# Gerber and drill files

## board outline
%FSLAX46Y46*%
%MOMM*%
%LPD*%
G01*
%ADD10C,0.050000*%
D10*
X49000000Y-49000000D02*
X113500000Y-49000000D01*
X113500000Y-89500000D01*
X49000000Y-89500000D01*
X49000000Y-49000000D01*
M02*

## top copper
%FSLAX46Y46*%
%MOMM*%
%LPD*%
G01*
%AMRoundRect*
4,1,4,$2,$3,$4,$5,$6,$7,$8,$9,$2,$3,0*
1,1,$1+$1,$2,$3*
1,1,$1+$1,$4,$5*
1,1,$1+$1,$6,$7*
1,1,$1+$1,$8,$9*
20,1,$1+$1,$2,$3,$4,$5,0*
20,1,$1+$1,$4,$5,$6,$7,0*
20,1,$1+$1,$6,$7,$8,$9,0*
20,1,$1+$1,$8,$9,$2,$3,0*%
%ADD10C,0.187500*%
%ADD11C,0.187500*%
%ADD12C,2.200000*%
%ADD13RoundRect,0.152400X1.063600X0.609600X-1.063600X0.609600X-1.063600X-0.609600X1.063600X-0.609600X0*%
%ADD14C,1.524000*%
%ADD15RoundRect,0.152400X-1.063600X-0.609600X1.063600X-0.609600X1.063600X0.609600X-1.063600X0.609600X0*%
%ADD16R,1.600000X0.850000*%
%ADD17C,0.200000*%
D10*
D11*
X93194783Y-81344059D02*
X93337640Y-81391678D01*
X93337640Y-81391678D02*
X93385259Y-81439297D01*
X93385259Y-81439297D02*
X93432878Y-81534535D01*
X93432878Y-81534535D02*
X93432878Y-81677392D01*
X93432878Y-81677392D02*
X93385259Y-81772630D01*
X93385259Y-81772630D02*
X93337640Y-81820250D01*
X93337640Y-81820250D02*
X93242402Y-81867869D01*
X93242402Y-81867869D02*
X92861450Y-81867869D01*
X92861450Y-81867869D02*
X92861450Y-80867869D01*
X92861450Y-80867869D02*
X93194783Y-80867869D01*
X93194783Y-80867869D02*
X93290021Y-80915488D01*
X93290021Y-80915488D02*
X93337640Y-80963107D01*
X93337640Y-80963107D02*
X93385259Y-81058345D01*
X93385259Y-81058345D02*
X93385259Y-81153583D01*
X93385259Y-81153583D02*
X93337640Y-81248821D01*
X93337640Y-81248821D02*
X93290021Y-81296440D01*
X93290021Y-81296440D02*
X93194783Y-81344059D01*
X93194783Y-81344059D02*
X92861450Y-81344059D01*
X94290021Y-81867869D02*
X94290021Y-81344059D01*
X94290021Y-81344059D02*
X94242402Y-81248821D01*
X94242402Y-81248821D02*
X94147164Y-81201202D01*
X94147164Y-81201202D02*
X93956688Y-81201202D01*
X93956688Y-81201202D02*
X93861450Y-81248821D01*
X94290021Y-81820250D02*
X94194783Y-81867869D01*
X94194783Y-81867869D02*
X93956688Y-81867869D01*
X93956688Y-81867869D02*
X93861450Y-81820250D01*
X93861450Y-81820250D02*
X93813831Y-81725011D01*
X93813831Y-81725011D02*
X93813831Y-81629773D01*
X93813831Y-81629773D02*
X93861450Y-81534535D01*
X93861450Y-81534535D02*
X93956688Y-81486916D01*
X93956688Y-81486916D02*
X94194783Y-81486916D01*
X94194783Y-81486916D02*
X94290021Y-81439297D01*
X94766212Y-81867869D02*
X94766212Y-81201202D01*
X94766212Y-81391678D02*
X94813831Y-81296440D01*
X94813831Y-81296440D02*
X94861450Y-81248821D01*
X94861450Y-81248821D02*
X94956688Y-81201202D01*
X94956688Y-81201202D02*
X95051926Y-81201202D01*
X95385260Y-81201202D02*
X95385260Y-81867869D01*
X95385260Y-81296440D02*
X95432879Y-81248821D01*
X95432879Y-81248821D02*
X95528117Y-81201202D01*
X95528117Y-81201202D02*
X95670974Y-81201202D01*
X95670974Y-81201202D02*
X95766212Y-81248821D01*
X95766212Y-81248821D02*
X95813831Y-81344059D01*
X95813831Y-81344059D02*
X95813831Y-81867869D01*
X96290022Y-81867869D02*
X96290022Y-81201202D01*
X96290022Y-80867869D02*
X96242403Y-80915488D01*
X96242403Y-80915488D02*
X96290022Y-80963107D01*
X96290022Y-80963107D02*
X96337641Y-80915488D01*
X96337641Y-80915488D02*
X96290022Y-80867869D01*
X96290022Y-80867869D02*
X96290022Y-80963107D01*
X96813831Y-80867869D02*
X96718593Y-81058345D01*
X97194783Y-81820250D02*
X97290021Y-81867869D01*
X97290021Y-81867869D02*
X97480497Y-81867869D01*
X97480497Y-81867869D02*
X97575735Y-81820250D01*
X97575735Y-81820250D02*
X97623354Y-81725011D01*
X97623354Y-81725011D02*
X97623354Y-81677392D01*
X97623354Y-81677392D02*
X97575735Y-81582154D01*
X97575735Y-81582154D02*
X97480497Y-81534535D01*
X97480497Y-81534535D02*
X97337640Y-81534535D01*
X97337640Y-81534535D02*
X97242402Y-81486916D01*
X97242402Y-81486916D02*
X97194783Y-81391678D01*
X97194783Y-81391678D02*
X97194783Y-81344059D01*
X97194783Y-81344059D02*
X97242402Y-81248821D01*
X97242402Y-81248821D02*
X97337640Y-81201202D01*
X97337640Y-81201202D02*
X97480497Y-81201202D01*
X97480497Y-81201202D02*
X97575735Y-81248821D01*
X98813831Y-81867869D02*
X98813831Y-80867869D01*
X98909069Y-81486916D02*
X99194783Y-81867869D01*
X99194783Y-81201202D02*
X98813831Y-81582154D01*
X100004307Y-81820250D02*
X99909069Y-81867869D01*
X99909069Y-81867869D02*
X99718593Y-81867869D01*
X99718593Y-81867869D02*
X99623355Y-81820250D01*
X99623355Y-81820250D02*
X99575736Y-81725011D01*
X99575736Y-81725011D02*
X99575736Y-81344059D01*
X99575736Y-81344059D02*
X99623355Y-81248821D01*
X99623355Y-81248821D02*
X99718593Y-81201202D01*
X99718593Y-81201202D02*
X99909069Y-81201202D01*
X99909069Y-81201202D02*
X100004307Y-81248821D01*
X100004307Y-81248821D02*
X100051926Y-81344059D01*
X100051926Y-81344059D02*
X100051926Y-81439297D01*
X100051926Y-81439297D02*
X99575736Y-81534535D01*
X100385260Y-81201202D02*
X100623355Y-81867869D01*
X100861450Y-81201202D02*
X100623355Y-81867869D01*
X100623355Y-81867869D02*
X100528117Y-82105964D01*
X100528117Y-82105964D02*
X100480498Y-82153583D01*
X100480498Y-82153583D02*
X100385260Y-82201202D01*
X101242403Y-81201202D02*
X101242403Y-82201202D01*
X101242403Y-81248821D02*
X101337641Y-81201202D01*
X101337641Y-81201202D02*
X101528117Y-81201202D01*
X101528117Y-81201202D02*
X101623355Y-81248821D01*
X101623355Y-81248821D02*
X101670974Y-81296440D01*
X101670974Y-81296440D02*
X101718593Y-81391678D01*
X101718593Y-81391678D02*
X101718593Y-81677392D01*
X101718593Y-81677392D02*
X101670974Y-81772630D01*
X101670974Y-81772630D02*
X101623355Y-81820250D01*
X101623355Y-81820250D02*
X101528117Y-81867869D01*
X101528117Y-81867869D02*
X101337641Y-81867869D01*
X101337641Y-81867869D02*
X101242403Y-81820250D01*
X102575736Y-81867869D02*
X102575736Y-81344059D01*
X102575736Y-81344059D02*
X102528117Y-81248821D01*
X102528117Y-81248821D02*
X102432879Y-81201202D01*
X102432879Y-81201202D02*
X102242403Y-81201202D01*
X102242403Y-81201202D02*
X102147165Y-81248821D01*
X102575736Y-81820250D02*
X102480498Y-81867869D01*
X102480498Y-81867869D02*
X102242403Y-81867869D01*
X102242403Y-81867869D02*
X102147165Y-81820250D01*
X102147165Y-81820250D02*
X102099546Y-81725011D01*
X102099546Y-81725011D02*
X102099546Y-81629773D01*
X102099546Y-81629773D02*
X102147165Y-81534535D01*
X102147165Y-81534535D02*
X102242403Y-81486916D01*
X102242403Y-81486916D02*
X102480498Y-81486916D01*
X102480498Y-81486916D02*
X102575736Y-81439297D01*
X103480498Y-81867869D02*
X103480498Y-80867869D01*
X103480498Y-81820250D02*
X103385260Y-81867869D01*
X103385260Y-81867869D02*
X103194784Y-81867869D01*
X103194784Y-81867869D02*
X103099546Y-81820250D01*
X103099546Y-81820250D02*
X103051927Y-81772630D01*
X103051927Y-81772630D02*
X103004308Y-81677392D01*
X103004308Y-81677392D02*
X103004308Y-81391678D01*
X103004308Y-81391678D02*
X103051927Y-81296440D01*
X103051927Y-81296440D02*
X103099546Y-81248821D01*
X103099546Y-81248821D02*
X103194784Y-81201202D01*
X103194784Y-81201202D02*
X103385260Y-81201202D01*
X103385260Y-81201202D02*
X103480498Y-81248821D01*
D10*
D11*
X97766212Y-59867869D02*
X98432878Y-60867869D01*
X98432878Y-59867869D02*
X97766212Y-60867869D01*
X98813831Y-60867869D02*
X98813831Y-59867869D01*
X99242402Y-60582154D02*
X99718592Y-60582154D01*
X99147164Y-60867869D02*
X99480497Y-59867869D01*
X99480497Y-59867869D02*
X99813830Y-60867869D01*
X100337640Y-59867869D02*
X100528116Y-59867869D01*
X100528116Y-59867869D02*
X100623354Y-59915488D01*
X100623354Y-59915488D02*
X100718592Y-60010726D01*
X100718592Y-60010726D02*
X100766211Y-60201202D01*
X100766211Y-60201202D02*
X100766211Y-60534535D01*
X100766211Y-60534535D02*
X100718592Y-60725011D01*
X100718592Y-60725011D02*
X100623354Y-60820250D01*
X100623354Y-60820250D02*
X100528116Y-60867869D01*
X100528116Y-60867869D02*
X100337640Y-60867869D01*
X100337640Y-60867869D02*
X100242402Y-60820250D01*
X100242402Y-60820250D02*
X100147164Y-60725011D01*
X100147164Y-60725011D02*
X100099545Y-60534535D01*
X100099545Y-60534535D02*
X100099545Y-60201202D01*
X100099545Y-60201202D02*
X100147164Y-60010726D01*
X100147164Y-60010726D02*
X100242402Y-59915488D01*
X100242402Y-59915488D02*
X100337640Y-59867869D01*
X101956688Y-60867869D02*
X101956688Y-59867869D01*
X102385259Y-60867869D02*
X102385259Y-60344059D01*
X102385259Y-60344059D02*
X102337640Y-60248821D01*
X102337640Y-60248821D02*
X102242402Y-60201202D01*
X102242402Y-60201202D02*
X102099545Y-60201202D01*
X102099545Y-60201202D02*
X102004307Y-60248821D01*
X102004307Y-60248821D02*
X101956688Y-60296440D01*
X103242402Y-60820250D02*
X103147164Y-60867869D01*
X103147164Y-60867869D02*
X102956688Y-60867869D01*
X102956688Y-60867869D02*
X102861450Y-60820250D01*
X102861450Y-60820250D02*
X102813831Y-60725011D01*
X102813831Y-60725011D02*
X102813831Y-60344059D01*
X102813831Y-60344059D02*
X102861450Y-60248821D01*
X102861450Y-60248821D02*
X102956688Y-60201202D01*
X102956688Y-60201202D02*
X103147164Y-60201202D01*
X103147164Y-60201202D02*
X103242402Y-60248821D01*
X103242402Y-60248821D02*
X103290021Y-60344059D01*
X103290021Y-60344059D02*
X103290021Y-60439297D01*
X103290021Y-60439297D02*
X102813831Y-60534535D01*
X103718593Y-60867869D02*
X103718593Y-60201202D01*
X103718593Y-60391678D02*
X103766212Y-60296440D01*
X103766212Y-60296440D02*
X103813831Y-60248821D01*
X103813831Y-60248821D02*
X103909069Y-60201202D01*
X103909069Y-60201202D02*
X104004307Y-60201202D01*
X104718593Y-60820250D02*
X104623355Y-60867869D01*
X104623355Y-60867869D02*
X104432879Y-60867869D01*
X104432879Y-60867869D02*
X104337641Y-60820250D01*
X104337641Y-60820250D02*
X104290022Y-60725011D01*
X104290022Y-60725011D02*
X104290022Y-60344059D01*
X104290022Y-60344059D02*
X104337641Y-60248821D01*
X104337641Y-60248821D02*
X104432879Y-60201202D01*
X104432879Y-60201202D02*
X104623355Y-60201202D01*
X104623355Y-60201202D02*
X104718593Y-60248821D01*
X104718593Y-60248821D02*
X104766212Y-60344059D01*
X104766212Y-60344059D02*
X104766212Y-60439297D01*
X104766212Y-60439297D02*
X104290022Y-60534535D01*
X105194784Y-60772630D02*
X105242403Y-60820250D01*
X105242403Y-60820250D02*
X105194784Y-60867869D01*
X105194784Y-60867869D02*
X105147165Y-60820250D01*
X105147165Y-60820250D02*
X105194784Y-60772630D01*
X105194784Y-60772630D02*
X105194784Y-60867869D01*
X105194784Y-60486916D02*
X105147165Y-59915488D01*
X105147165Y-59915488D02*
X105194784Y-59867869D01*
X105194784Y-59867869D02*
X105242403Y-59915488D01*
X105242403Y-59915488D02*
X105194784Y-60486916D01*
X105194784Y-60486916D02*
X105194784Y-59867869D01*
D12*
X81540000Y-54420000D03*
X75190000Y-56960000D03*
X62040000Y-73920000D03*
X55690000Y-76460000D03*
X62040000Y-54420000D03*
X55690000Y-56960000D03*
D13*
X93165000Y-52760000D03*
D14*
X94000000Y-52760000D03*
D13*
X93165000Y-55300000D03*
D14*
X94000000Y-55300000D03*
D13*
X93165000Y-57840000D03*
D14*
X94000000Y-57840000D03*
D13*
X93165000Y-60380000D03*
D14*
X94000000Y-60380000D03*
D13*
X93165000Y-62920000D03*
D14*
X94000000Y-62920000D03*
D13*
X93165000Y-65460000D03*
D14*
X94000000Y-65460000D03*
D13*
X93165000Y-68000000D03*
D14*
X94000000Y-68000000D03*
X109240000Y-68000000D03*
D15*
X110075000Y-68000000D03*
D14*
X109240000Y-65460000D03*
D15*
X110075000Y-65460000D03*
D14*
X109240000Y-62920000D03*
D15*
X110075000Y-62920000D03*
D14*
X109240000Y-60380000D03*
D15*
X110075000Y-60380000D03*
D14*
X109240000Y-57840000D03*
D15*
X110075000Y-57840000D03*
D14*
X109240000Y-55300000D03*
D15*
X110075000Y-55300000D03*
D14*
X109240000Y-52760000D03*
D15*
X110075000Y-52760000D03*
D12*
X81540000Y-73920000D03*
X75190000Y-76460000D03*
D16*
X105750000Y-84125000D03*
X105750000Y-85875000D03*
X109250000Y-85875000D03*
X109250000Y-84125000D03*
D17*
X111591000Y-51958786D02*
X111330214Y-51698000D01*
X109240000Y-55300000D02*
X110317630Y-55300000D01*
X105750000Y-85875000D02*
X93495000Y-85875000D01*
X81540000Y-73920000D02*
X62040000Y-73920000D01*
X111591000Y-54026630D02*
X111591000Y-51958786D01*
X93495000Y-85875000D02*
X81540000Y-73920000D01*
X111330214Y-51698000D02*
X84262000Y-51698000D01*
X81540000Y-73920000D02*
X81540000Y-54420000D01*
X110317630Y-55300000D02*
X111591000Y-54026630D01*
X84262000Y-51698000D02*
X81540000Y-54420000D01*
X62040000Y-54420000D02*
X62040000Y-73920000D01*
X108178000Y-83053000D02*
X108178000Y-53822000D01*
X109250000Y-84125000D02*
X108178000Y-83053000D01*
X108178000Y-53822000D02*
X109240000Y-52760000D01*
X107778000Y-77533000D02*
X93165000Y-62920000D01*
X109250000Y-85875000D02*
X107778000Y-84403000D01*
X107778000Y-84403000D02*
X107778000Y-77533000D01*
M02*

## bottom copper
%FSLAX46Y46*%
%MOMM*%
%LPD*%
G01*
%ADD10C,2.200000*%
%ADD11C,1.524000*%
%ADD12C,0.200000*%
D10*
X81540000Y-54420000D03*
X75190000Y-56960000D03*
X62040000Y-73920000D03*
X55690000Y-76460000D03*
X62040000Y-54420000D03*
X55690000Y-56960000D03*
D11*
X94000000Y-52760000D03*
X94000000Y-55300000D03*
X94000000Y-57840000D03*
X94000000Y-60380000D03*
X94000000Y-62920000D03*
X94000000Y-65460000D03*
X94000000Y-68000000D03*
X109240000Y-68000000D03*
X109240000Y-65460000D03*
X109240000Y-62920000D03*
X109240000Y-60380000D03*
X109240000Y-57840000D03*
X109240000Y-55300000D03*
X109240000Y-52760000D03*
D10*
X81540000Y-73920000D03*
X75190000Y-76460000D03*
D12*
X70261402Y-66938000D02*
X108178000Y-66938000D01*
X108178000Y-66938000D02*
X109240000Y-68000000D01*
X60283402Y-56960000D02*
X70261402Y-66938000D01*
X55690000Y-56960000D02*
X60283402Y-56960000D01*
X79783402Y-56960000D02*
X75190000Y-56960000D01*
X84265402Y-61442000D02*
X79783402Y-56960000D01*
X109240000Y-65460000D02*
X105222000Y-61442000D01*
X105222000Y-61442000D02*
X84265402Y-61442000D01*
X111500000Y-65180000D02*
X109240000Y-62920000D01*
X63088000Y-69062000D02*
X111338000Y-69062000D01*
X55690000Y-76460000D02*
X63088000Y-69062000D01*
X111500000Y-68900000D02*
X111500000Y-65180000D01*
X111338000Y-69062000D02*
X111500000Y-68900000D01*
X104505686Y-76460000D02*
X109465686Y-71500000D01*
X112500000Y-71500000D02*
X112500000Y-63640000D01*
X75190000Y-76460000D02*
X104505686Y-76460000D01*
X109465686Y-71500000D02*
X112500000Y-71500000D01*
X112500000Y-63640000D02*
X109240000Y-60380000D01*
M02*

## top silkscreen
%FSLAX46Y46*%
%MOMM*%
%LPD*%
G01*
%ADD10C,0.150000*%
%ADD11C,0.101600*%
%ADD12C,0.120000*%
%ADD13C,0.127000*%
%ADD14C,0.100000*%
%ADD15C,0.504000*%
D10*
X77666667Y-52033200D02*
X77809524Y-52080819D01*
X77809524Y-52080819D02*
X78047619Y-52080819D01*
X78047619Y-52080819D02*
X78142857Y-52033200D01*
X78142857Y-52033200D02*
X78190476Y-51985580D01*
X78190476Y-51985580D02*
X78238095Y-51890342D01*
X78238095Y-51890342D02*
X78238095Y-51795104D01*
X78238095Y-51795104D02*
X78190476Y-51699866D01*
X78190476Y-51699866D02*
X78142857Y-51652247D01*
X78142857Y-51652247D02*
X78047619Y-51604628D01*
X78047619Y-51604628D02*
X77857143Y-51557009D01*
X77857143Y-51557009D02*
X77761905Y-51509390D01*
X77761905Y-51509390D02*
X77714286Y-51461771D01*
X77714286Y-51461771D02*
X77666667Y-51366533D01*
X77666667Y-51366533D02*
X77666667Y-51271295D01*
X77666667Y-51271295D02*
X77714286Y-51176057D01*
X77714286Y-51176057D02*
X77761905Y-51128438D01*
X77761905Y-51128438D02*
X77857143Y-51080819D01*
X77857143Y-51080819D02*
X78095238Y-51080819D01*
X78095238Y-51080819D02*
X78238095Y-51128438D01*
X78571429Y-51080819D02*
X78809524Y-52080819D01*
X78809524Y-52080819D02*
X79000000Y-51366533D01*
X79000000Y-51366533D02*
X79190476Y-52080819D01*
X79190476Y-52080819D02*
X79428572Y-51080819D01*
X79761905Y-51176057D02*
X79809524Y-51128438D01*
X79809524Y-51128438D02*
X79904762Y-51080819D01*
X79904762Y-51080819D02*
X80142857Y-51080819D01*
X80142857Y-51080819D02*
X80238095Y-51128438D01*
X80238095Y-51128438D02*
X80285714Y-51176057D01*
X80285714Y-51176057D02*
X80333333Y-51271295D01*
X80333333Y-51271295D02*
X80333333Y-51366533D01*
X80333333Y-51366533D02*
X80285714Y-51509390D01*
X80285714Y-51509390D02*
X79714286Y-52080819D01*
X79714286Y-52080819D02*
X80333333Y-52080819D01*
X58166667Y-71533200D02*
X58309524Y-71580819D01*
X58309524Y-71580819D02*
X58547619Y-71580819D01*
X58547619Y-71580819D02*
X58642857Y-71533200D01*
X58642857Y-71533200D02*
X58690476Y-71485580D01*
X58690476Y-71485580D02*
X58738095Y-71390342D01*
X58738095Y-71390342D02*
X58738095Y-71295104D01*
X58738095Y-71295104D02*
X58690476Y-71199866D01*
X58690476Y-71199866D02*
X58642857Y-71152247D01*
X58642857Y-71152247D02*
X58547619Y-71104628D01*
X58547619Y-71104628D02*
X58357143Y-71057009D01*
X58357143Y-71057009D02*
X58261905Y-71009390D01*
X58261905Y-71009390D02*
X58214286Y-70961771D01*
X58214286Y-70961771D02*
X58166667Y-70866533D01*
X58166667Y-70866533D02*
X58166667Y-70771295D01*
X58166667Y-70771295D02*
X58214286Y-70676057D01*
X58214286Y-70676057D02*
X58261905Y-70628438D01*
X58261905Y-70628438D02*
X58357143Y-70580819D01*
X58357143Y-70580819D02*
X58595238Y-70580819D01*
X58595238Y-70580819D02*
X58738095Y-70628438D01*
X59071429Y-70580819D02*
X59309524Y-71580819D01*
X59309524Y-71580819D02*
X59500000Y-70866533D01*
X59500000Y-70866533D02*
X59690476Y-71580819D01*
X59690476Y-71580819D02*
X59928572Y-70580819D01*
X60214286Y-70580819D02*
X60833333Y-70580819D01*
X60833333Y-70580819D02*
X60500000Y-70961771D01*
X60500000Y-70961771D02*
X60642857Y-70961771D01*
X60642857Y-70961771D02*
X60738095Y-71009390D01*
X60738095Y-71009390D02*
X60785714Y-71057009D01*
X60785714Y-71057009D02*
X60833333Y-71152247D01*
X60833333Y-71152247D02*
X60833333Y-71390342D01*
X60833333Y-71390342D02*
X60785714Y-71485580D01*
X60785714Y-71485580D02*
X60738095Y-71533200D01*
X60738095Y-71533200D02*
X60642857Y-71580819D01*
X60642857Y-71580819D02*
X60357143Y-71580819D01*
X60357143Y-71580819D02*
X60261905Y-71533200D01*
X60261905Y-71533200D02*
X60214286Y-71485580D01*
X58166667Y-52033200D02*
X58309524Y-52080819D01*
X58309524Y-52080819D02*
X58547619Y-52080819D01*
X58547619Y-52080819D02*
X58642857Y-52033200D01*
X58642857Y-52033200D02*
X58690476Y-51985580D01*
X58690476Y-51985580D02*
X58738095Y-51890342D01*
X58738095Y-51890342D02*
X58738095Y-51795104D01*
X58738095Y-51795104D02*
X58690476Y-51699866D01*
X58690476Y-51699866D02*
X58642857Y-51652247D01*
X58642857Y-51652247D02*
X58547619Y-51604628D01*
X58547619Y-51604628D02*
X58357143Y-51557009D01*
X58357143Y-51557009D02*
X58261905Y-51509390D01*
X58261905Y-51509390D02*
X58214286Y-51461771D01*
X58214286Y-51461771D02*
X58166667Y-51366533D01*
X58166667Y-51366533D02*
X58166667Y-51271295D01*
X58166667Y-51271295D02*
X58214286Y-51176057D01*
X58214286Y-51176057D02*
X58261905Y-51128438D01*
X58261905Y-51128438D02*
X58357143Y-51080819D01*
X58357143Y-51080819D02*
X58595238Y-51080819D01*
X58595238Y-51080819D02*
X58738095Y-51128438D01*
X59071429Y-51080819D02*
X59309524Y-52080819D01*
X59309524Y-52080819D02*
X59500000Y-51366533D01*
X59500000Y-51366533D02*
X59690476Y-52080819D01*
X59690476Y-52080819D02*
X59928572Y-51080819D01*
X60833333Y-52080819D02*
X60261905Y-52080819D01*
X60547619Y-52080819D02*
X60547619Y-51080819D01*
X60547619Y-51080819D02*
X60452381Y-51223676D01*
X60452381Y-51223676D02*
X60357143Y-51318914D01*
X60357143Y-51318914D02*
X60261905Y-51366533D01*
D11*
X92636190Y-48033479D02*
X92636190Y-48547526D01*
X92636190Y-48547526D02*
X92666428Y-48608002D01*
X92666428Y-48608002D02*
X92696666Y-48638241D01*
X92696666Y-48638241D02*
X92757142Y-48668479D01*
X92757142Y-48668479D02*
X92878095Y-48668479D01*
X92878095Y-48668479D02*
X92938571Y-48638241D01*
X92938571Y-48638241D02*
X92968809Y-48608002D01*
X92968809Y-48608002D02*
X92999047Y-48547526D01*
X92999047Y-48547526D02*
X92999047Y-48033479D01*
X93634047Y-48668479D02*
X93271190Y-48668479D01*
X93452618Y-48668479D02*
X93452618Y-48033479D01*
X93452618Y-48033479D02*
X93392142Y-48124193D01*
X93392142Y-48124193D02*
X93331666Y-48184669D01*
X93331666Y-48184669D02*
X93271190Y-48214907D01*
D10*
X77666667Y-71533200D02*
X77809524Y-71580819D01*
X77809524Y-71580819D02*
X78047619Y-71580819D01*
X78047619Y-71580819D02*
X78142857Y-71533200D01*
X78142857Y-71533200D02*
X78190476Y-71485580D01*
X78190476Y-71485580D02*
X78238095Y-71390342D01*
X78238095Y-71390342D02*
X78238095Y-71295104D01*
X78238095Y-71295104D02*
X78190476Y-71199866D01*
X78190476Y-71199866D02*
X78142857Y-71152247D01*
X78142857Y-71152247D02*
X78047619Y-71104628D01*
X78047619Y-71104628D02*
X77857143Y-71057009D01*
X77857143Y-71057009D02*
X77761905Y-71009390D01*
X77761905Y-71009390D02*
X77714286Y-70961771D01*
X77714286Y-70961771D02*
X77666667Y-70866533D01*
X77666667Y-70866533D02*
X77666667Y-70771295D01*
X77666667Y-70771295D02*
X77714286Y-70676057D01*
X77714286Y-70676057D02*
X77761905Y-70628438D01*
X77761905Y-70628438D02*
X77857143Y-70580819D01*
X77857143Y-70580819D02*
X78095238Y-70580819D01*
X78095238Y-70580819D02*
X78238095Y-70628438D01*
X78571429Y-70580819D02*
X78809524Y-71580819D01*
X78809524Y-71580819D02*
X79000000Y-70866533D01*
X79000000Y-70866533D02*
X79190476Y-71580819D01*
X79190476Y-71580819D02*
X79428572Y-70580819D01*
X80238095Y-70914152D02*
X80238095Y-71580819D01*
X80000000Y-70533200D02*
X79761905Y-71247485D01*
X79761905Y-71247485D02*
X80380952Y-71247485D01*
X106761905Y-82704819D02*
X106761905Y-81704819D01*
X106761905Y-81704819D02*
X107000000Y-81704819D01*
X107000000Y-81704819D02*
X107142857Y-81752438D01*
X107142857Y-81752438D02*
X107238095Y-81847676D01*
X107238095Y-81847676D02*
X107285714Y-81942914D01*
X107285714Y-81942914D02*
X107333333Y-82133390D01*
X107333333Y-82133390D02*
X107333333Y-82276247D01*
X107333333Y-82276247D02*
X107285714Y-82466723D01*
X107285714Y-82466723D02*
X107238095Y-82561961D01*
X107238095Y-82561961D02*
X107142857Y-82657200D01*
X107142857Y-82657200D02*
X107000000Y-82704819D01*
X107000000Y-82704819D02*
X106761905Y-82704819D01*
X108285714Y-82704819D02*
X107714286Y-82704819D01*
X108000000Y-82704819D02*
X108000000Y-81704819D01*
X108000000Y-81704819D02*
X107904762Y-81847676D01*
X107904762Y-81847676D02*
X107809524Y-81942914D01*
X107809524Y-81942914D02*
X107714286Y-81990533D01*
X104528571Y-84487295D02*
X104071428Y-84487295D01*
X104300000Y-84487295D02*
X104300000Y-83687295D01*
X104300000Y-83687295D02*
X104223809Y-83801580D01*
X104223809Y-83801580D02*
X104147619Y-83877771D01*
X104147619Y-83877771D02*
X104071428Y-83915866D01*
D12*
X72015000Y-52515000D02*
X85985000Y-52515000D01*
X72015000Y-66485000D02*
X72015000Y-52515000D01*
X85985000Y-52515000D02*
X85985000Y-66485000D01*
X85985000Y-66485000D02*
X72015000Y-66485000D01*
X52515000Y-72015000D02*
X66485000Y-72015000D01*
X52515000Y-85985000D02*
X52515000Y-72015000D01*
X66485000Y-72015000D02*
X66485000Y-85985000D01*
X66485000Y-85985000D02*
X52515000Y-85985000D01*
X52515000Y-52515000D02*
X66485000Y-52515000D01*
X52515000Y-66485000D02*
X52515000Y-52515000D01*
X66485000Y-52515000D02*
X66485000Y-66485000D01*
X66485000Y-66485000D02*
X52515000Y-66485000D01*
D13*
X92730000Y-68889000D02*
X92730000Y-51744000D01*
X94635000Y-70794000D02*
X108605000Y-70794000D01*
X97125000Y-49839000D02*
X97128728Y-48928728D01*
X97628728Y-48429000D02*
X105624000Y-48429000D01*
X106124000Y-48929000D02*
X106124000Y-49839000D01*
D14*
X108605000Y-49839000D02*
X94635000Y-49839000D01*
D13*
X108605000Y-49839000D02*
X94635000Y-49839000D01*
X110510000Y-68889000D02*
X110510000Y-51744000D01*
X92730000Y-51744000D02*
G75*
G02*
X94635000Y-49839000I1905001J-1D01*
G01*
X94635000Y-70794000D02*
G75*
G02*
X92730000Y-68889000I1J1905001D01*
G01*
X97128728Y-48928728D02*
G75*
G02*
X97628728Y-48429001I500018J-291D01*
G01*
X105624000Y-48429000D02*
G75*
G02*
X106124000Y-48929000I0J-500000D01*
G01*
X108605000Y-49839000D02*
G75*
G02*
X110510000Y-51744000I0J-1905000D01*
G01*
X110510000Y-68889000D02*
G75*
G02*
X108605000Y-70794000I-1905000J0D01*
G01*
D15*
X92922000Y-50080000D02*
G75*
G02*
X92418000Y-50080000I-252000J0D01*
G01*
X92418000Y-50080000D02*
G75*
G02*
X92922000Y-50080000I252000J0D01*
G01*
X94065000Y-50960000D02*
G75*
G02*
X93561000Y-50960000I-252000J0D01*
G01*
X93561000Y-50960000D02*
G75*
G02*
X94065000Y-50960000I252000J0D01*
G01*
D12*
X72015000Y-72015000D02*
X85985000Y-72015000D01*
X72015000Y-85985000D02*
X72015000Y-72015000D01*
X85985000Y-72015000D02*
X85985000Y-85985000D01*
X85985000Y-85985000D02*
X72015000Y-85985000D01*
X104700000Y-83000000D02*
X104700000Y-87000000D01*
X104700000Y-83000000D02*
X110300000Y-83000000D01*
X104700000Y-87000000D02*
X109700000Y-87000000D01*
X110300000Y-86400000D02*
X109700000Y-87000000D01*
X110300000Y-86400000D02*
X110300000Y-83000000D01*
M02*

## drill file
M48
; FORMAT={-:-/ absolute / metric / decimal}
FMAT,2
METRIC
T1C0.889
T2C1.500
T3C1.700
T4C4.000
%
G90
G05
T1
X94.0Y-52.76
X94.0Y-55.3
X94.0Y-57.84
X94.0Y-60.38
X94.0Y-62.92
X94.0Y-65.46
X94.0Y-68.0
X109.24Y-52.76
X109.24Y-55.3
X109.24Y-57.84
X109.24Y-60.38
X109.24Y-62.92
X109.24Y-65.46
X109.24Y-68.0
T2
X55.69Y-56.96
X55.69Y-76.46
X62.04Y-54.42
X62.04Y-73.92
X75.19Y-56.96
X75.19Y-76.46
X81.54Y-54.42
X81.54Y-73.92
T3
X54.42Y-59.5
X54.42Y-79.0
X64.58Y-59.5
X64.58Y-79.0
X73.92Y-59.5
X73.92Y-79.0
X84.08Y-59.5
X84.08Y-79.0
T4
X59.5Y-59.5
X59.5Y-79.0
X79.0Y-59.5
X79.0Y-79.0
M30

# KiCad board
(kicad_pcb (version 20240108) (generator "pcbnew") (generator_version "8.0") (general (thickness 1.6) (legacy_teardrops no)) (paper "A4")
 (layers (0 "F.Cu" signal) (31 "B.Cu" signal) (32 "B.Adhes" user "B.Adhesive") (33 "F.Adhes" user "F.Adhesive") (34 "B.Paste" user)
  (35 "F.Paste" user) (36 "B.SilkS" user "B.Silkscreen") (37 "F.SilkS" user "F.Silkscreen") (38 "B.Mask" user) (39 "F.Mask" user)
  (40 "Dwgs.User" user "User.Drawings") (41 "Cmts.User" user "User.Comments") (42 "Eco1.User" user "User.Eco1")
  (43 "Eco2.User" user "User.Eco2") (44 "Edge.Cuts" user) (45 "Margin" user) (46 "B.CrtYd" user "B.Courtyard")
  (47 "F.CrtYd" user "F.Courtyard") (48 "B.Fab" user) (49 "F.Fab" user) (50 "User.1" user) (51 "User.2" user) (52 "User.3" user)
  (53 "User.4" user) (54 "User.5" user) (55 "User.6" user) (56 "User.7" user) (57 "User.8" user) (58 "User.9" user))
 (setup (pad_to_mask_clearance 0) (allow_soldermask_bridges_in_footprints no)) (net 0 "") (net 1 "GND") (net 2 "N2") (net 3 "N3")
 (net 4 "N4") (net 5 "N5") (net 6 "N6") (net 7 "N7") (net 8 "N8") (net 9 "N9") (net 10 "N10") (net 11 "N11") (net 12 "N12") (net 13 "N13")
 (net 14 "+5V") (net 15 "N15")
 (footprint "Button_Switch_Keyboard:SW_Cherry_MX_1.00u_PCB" (layer "F.Cu") (at 81.54 54.42)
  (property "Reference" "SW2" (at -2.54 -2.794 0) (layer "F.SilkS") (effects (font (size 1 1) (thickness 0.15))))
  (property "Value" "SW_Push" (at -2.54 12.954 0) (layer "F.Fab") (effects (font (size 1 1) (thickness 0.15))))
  (fp_line (start -9.525 -1.905) (end 4.445 -1.905) (stroke (width 0.12) (type solid)) (layer "F.SilkS"))
  (fp_line (start -9.525 12.065) (end -9.525 -1.905) (stroke (width 0.12) (type solid)) (layer "F.SilkS"))
  (fp_line (start 4.445 -1.905) (end 4.445 12.065) (stroke (width 0.12) (type solid)) (layer "F.SilkS"))
  (fp_line (start 4.445 12.065) (end -9.525 12.065) (stroke (width 0.12) (type solid)) (layer "F.SilkS"))
  (pad "" np_thru_hole circle (at -7.62 5.08) (size 1.7 1.7) (drill 1.7) (layers "*.Cu" "*.Mask"))
  (pad "" np_thru_hole circle (at -2.54 5.08) (size 4 4) (drill 4) (layers "*.Cu" "*.Mask"))
  (pad "" np_thru_hole circle (at 2.54 5.08) (size 1.7 1.7) (drill 1.7) (layers "*.Cu" "*.Mask"))
  (pad "1" thru_hole circle (at 0 0) (size 2.2 2.2) (drill 1.5) (layers "*.Cu" "*.Mask") (remove_unused_layers no) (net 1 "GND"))
  (pad "2" thru_hole circle (at -6.35 2.54) (size 2.2 2.2) (drill 1.5) (layers "*.Cu" "*.Mask") (remove_unused_layers no) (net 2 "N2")))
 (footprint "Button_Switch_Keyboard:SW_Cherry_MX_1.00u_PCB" (layer "F.Cu") (at 62.04 73.92)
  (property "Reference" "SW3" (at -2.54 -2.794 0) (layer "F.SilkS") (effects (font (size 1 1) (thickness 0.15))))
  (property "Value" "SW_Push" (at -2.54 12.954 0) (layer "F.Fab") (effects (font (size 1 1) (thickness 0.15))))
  (fp_line (start -9.525 -1.905) (end 4.445 -1.905) (stroke (width 0.12) (type solid)) (layer "F.SilkS"))
  (fp_line (start -9.525 12.065) (end -9.525 -1.905) (stroke (width 0.12) (type solid)) (layer "F.SilkS"))
  (fp_line (start 4.445 -1.905) (end 4.445 12.065) (stroke (width 0.12) (type solid)) (layer "F.SilkS"))
  (fp_line (start 4.445 12.065) (end -9.525 12.065) (stroke (width 0.12) (type solid)) (layer "F.SilkS"))
  (pad "" np_thru_hole circle (at -7.62 5.08) (size 1.7 1.7) (drill 1.7) (layers "*.Cu" "*.Mask"))
  (pad "" np_thru_hole circle (at -2.54 5.08) (size 4 4) (drill 4) (layers "*.Cu" "*.Mask"))
  (pad "" np_thru_hole circle (at 2.54 5.08) (size 1.7 1.7) (drill 1.7) (layers "*.Cu" "*.Mask"))
  (pad "1" thru_hole circle (at 0 0) (size 2.2 2.2) (drill 1.5) (layers "*.Cu" "*.Mask") (remove_unused_layers no) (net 1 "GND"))
  (pad "2" thru_hole circle (at -6.35 2.54) (size 2.2 2.2) (drill 1.5) (layers "*.Cu" "*.Mask") (remove_unused_layers no) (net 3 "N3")))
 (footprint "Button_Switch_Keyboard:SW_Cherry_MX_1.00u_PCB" (layer "F.Cu") (at 62.04 54.42)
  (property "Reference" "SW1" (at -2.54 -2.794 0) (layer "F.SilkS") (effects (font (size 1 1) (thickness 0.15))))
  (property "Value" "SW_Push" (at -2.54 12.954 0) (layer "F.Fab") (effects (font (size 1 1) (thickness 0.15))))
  (fp_line (start -9.525 -1.905) (end 4.445 -1.905) (stroke (width 0.12) (type solid)) (layer "F.SilkS"))
  (fp_line (start -9.525 12.065) (end -9.525 -1.905) (stroke (width 0.12) (type solid)) (layer "F.SilkS"))
  (fp_line (start 4.445 -1.905) (end 4.445 12.065) (stroke (width 0.12) (type solid)) (layer "F.SilkS"))
  (fp_line (start 4.445 12.065) (end -9.525 12.065) (stroke (width 0.12) (type solid)) (layer "F.SilkS"))
  (pad "" np_thru_hole circle (at -7.62 5.08) (size 1.7 1.7) (drill 1.7) (layers "*.Cu" "*.Mask"))
  (pad "" np_thru_hole circle (at -2.54 5.08) (size 4 4) (drill 4) (layers "*.Cu" "*.Mask"))
  (pad "" np_thru_hole circle (at 2.54 5.08) (size 1.7 1.7) (drill 1.7) (layers "*.Cu" "*.Mask"))
  (pad "1" thru_hole circle (at 0 0) (size 2.2 2.2) (drill 1.5) (layers "*.Cu" "*.Mask") (remove_unused_layers no) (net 1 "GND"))
  (pad "2" thru_hole circle (at -6.35 2.54) (size 2.2 2.2) (drill 1.5) (layers "*.Cu" "*.Mask") (remove_unused_layers no) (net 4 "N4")))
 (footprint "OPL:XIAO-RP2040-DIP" (layer "F.Cu") (at 101.62 60.38)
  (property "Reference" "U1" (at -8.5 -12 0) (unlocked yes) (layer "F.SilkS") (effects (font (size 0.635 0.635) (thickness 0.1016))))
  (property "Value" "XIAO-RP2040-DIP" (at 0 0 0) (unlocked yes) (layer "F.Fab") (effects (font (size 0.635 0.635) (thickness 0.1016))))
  (fp_line (start -8.89 8.509) (end -8.89 -8.636) (stroke (width 0.127) (type solid)) (layer "F.SilkS"))
  (fp_line (start -6.985 10.414) (end 6.985 10.414) (stroke (width 0.127) (type solid)) (layer "F.SilkS"))
  (fp_line (start -4.495 -10.541) (end -4.491272 -11.451272) (stroke (width 0.127) (type solid)) (layer "F.SilkS"))
  (fp_line (start -3.991272 -11.951) (end 4.004 -11.951) (stroke (width 0.127) (type solid)) (layer "F.SilkS"))
  (fp_line (start 4.504 -11.451) (end 4.504 -10.541) (stroke (width 0.127) (type solid)) (layer "F.SilkS"))
  (fp_line (start 6.985 -10.541) (end -6.985 -10.541) (stroke (width 0.1) (type solid)) (layer "F.SilkS"))
  (fp_line (start 6.985 -10.541) (end -6.985 -10.541) (stroke (width 0.127) (type solid)) (layer "F.SilkS"))
  (fp_line (start 8.89 8.509) (end 8.89 -8.636) (stroke (width 0.127) (type solid)) (layer "F.SilkS"))
  (fp_arc (start -8.89 -8.636) (mid -8.332038 -9.983038) (end -6.985 -10.541) (stroke (width 0.127) (type solid)) (layer "F.SilkS"))
  (fp_arc (start -6.985 10.414) (mid -8.332038 9.856038) (end -8.89 8.509) (stroke (width 0.127) (type solid)) (layer "F.SilkS"))
  (fp_arc (start -4.491272 -11.451272) (mid -4.344724 -11.804644) (end -3.991272 -11.951) (stroke (width 0.127) (type default))
   (layer "F.SilkS"))
  (fp_arc (start 4.004 -11.951) (mid 4.357553 -11.804553) (end 4.504 -11.451) (stroke (width 0.127) (type default)) (layer "F.SilkS"))
  (fp_arc (start 6.985 -10.541) (mid 8.332038 -9.983038) (end 8.89 -8.636) (stroke (width 0.127) (type solid)) (layer "F.SilkS"))
  (fp_arc (start 8.89 8.509) (mid 8.332038 9.856038) (end 6.985 10.414) (stroke (width 0.127) (type solid)) (layer "F.SilkS"))
  (fp_circle (center -8.95 -10.3) (end -8.95 -10.554) (stroke (width 0.5) (type solid)) (fill solid) (layer "F.SilkS"))
  (fp_circle (center -7.807 -9.42) (end -7.807 -9.674) (stroke (width 0.5) (type solid)) (fill solid) (layer "F.SilkS"))
  (pad "1" smd roundrect (at -8.455 -7.62 180) (size 2.432 1.524) (layers "F.Cu" "F.Mask") (roundrect_rratio 0.1) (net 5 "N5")
   (thermal_bridge_angle 45))
  (pad "1" thru_hole circle (at -7.62 -7.62 180) (size 1.524 1.524) (drill 0.889) (layers "*.Cu" "*.Mask") (remove_unused_layers no)
   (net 5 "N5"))
  (pad "2" smd roundrect (at -8.455 -5.08 180) (size 2.432 1.524) (layers "F.Cu" "F.Mask") (roundrect_rratio 0.1) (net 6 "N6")
   (thermal_bridge_angle 45))
  (pad "2" thru_hole circle (at -7.62 -5.08 180) (size 1.524 1.524) (drill 0.889) (layers "*.Cu" "*.Mask") (remove_unused_layers no)
   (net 6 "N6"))
  (pad "3" smd roundrect (at -8.455 -2.54 180) (size 2.432 1.524) (layers "F.Cu" "F.Mask") (roundrect_rratio 0.1) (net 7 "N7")
   (thermal_bridge_angle 45))
  (pad "3" thru_hole circle (at -7.62 -2.54 180) (size 1.524 1.524) (drill 0.889) (layers "*.Cu" "*.Mask") (remove_unused_layers no)
   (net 7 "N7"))
  (pad "4" smd roundrect (at -8.455 0 180) (size 2.432 1.524) (layers "F.Cu" "F.Mask") (roundrect_rratio 0.1) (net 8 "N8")
   (thermal_bridge_angle 45))
  (pad "4" thru_hole circle (at -7.62 0 180) (size 1.524 1.524) (drill 0.889) (layers "*.Cu" "*.Mask") (remove_unused_layers no)
   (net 8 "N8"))
  (pad "5" smd roundrect (at -8.455 2.54 180) (size 2.432 1.524) (layers "F.Cu" "F.Mask") (roundrect_rratio 0.1) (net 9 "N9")
   (thermal_bridge_angle 45))
  (pad "5" thru_hole circle (at -7.62 2.54 180) (size 1.524 1.524) (drill 0.889) (layers "*.Cu" "*.Mask") (remove_unused_layers no)
   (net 9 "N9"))
  (pad "6" smd roundrect (at -8.455 5.08 180) (size 2.432 1.524) (layers "F.Cu" "F.Mask") (roundrect_rratio 0.1) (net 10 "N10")
   (thermal_bridge_angle 45))
  (pad "6" thru_hole circle (at -7.62 5.08 180) (size 1.524 1.524) (drill 0.889) (layers "*.Cu" "*.Mask") (remove_unused_layers no)
   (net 10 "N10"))
  (pad "7" smd roundrect (at -8.455 7.62 180) (size 2.432 1.524) (layers "F.Cu" "F.Mask") (roundrect_rratio 0.1) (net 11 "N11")
   (thermal_bridge_angle 45))
  (pad "7" thru_hole circle (at -7.62 7.62 180) (size 1.524 1.524) (drill 0.889) (layers "*.Cu" "*.Mask") (remove_unused_layers no)
   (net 11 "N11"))
  (pad "8" thru_hole circle (at 7.62 7.62) (size 1.524 1.524) (drill 0.889) (layers "*.Cu" "*.Mask") (remove_unused_layers no) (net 4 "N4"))
  (pad "8" smd roundrect (at 8.455 7.62) (size 2.432 1.524) (layers "F.Cu" "F.Mask") (roundrect_rratio 0.1) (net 4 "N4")
   (thermal_bridge_angle 45))
  (pad "9" thru_hole circle (at 7.62 5.08) (size 1.524 1.524) (drill 0.889) (layers "*.Cu" "*.Mask") (remove_unused_layers no) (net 2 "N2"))
  (pad "9" smd roundrect (at 8.455 5.08) (size 2.432 1.524) (layers "F.Cu" "F.Mask") (roundrect_rratio 0.1) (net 2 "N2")
   (thermal_bridge_angle 45))
  (pad "10" thru_hole circle (at 7.62 2.54) (size 1.524 1.524) (drill 0.889) (layers "*.Cu" "*.Mask") (remove_unused_layers no) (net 3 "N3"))
  (pad "10" smd roundrect (at 8.455 2.54) (size 2.432 1.524) (layers "F.Cu" "F.Mask") (roundrect_rratio 0.1) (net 3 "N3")
   (thermal_bridge_angle 45))
  (pad "11" thru_hole circle (at 7.62 0) (size 1.524 1.524) (drill 0.889) (layers "*.Cu" "*.Mask") (remove_unused_layers no) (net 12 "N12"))
  (pad "11" smd roundrect (at 8.455 0) (size 2.432 1.524) (layers "F.Cu" "F.Mask") (roundrect_rratio 0.1) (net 12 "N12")
   (thermal_bridge_angle 45))
  (pad "12" thru_hole circle (at 7.62 -2.54) (size 1.524 1.524) (drill 0.889) (layers "*.Cu" "*.Mask") (remove_unused_layers no)
   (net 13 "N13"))
  (pad "12" smd roundrect (at 8.455 -2.54) (size 2.432 1.524) (layers "F.Cu" "F.Mask") (roundrect_rratio 0.1) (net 13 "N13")
   (thermal_bridge_angle 45))
  (pad "13" thru_hole circle (at 7.62 -5.08) (size 1.524 1.524) (drill 0.889) (layers "*.Cu" "*.Mask") (remove_unused_layers no)
   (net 1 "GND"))
  (pad "13" smd roundrect (at 8.455 -5.08) (size 2.432 1.524) (layers "F.Cu" "F.Mask") (roundrect_rratio 0.1) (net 1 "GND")
   (thermal_bridge_angle 45))
  (pad "14" thru_hole circle (at 7.62 -7.62) (size 1.524 1.524) (drill 0.889) (layers "*.Cu" "*.Mask") (remove_unused_layers no)
   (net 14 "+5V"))
  (pad "14" smd roundrect (at 8.455 -7.62) (size 2.432 1.524) (layers "F.Cu" "F.Mask") (roundrect_rratio 0.1) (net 14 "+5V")
   (thermal_bridge_angle 45)))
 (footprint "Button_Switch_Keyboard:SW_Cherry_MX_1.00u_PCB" (layer "F.Cu") (at 81.54 73.92)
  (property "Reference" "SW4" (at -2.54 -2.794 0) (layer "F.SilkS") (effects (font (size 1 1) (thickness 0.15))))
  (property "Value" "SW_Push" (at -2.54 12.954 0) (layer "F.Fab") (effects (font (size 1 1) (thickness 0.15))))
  (fp_line (start -9.525 -1.905) (end 4.445 -1.905) (stroke (width 0.12) (type solid)) (layer "F.SilkS"))
  (fp_line (start -9.525 12.065) (end -9.525 -1.905) (stroke (width 0.12) (type solid)) (layer "F.SilkS"))
  (fp_line (start 4.445 -1.905) (end 4.445 12.065) (stroke (width 0.12) (type solid)) (layer "F.SilkS"))
  (fp_line (start 4.445 12.065) (end -9.525 12.065) (stroke (width 0.12) (type solid)) (layer "F.SilkS"))
  (pad "" np_thru_hole circle (at -7.62 5.08) (size 1.7 1.7) (drill 1.7) (layers "*.Cu" "*.Mask"))
  (pad "" np_thru_hole circle (at -2.54 5.08) (size 4 4) (drill 4) (layers "*.Cu" "*.Mask"))
  (pad "" np_thru_hole circle (at 2.54 5.08) (size 1.7 1.7) (drill 1.7) (layers "*.Cu" "*.Mask"))
  (pad "1" thru_hole circle (at 0 0) (size 2.2 2.2) (drill 1.5) (layers "*.Cu" "*.Mask") (remove_unused_layers no) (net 1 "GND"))
  (pad "2" thru_hole circle (at -6.35 2.54) (size 2.2 2.2) (drill 1.5) (layers "*.Cu" "*.Mask") (remove_unused_layers no) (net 12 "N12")))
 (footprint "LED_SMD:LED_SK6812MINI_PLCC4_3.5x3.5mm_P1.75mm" (layer "F.Cu") (at 107.5 85)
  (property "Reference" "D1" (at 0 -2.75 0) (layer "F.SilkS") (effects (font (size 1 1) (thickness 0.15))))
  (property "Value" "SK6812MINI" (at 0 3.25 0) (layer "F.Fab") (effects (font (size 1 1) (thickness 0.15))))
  (fp_line (start -2.8 -2) (end -2.8 2) (stroke (width 0.12) (type default)) (layer "F.SilkS"))
  (fp_line (start -2.8 -2) (end 2.8 -2) (stroke (width 0.12) (type solid)) (layer "F.SilkS"))
  (fp_line (start -2.8 2) (end 2.2 2) (stroke (width 0.12) (type solid)) (layer "F.SilkS"))
  (fp_line (start 2.8 1.4) (end 2.2 2) (stroke (width 0.12) (type default)) (layer "F.SilkS"))
  (fp_line (start 2.8 1.4) (end 2.8 -2) (stroke (width 0.12) (type solid)) (layer "F.SilkS"))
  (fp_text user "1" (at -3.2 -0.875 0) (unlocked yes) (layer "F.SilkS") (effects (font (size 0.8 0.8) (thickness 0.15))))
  (pad "1" smd rect (at -1.75 -0.875) (size 1.6 0.85) (layers "F.Cu" "F.Paste" "F.Mask") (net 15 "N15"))
  (pad "2" smd rect (at -1.75 0.875) (size 1.6 0.85) (layers "F.Cu" "F.Paste" "F.Mask") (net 1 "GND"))
  (pad "3" smd rect (at 1.75 0.875) (size 1.6 0.85) (layers "F.Cu" "F.Paste" "F.Mask") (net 9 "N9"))
  (pad "4" smd rect (at 1.75 -0.875) (size 1.6 0.85) (layers "F.Cu" "F.Paste" "F.Mask") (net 14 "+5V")))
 (gr_rect (start 49 49) (end 113.5 89.5) (stroke (width 0.05) (type default)) (fill none) (layer "Edge.Cuts"))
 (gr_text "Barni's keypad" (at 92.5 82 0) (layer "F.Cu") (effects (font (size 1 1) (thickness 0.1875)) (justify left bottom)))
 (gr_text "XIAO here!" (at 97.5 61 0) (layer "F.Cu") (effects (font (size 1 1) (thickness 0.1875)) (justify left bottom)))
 (segment (start 111.591 51.958786) (end 111.330214 51.698) (width 0.2) (layer "F.Cu") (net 1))
 (segment (start 109.24 55.3) (end 110.31763 55.3) (width 0.2) (layer "F.Cu") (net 1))
 (segment (start 105.75 85.875) (end 93.495 85.875) (width 0.2) (layer "F.Cu") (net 1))
 (segment (start 81.54 73.92) (end 62.04 73.92) (width 0.2) (layer "F.Cu") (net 1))
 (segment (start 111.591 54.02663) (end 111.591 51.958786) (width 0.2) (layer "F.Cu") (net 1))
 (segment (start 93.495 85.875) (end 81.54 73.92) (width 0.2) (layer "F.Cu") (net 1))
 (segment (start 111.330214 51.698) (end 84.262 51.698) (width 0.2) (layer "F.Cu") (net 1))
 (segment (start 81.54 73.92) (end 81.54 54.42) (width 0.2) (layer "F.Cu") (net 1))
 (segment (start 110.31763 55.3) (end 111.591 54.02663) (width 0.2) (layer "F.Cu") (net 1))
 (segment (start 84.262 51.698) (end 81.54 54.42) (width 0.2) (layer "F.Cu") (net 1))
 (segment (start 62.04 54.42) (end 62.04 73.92) (width 0.2) (layer "F.Cu") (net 1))
 (segment (start 108.178 83.053) (end 108.178 53.822) (width 0.2) (layer "F.Cu") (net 14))
 (segment (start 109.25 84.125) (end 108.178 83.053) (width 0.2) (layer "F.Cu") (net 14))
 (segment (start 108.178 53.822) (end 109.24 52.76) (width 0.2) (layer "F.Cu") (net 14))
 (segment (start 107.778 77.533) (end 93.165 62.92) (width 0.2) (layer "F.Cu") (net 9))
 (segment (start 109.25 85.875) (end 107.778 84.403) (width 0.2) (layer "F.Cu") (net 9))
 (segment (start 107.778 84.403) (end 107.778 77.533) (width 0.2) (layer "F.Cu") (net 9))
 (segment (start 70.261402 66.938) (end 108.178 66.938) (width 0.2) (layer "B.Cu") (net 4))
 (segment (start 108.178 66.938) (end 109.24 68) (width 0.2) (layer "B.Cu") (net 4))
 (segment (start 60.283402 56.96) (end 70.261402 66.938) (width 0.2) (layer "B.Cu") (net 4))
 (segment (start 55.69 56.96) (end 60.283402 56.96) (width 0.2) (layer "B.Cu") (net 4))
 (segment (start 79.783402 56.96) (end 75.19 56.96) (width 0.2) (layer "B.Cu") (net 2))
 (segment (start 84.265402 61.442) (end 79.783402 56.96) (width 0.2) (layer "B.Cu") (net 2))
 (segment (start 109.24 65.46) (end 105.222 61.442) (width 0.2) (layer "B.Cu") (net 2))
 (segment (start 105.222 61.442) (end 84.265402 61.442) (width 0.2) (layer "B.Cu") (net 2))
 (segment (start 111.5 65.18) (end 109.24 62.92) (width 0.2) (layer "B.Cu") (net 3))
 (segment (start 63.088 69.062) (end 111.338 69.062) (width 0.2) (layer "B.Cu") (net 3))
 (segment (start 55.69 76.46) (end 63.088 69.062) (width 0.2) (layer "B.Cu") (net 3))
 (segment (start 111.5 68.9) (end 111.5 65.18) (width 0.2) (layer "B.Cu") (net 3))
 (segment (start 111.338 69.062) (end 111.5 68.9) (width 0.2) (layer "B.Cu") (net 3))
 (segment (start 104.505686 76.46) (end 109.465686 71.5) (width 0.2) (layer "B.Cu") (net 12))
 (segment (start 112.5 71.5) (end 112.5 63.64) (width 0.2) (layer "B.Cu") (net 12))
 (segment (start 75.19 76.46) (end 104.505686 76.46) (width 0.2) (layer "B.Cu") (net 12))
 (segment (start 109.465686 71.5) (end 112.5 71.5) (width 0.2) (layer "B.Cu") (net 12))
 (segment (start 112.5 63.64) (end 109.24 60.38) (width 0.2) (layer "B.Cu") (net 12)))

